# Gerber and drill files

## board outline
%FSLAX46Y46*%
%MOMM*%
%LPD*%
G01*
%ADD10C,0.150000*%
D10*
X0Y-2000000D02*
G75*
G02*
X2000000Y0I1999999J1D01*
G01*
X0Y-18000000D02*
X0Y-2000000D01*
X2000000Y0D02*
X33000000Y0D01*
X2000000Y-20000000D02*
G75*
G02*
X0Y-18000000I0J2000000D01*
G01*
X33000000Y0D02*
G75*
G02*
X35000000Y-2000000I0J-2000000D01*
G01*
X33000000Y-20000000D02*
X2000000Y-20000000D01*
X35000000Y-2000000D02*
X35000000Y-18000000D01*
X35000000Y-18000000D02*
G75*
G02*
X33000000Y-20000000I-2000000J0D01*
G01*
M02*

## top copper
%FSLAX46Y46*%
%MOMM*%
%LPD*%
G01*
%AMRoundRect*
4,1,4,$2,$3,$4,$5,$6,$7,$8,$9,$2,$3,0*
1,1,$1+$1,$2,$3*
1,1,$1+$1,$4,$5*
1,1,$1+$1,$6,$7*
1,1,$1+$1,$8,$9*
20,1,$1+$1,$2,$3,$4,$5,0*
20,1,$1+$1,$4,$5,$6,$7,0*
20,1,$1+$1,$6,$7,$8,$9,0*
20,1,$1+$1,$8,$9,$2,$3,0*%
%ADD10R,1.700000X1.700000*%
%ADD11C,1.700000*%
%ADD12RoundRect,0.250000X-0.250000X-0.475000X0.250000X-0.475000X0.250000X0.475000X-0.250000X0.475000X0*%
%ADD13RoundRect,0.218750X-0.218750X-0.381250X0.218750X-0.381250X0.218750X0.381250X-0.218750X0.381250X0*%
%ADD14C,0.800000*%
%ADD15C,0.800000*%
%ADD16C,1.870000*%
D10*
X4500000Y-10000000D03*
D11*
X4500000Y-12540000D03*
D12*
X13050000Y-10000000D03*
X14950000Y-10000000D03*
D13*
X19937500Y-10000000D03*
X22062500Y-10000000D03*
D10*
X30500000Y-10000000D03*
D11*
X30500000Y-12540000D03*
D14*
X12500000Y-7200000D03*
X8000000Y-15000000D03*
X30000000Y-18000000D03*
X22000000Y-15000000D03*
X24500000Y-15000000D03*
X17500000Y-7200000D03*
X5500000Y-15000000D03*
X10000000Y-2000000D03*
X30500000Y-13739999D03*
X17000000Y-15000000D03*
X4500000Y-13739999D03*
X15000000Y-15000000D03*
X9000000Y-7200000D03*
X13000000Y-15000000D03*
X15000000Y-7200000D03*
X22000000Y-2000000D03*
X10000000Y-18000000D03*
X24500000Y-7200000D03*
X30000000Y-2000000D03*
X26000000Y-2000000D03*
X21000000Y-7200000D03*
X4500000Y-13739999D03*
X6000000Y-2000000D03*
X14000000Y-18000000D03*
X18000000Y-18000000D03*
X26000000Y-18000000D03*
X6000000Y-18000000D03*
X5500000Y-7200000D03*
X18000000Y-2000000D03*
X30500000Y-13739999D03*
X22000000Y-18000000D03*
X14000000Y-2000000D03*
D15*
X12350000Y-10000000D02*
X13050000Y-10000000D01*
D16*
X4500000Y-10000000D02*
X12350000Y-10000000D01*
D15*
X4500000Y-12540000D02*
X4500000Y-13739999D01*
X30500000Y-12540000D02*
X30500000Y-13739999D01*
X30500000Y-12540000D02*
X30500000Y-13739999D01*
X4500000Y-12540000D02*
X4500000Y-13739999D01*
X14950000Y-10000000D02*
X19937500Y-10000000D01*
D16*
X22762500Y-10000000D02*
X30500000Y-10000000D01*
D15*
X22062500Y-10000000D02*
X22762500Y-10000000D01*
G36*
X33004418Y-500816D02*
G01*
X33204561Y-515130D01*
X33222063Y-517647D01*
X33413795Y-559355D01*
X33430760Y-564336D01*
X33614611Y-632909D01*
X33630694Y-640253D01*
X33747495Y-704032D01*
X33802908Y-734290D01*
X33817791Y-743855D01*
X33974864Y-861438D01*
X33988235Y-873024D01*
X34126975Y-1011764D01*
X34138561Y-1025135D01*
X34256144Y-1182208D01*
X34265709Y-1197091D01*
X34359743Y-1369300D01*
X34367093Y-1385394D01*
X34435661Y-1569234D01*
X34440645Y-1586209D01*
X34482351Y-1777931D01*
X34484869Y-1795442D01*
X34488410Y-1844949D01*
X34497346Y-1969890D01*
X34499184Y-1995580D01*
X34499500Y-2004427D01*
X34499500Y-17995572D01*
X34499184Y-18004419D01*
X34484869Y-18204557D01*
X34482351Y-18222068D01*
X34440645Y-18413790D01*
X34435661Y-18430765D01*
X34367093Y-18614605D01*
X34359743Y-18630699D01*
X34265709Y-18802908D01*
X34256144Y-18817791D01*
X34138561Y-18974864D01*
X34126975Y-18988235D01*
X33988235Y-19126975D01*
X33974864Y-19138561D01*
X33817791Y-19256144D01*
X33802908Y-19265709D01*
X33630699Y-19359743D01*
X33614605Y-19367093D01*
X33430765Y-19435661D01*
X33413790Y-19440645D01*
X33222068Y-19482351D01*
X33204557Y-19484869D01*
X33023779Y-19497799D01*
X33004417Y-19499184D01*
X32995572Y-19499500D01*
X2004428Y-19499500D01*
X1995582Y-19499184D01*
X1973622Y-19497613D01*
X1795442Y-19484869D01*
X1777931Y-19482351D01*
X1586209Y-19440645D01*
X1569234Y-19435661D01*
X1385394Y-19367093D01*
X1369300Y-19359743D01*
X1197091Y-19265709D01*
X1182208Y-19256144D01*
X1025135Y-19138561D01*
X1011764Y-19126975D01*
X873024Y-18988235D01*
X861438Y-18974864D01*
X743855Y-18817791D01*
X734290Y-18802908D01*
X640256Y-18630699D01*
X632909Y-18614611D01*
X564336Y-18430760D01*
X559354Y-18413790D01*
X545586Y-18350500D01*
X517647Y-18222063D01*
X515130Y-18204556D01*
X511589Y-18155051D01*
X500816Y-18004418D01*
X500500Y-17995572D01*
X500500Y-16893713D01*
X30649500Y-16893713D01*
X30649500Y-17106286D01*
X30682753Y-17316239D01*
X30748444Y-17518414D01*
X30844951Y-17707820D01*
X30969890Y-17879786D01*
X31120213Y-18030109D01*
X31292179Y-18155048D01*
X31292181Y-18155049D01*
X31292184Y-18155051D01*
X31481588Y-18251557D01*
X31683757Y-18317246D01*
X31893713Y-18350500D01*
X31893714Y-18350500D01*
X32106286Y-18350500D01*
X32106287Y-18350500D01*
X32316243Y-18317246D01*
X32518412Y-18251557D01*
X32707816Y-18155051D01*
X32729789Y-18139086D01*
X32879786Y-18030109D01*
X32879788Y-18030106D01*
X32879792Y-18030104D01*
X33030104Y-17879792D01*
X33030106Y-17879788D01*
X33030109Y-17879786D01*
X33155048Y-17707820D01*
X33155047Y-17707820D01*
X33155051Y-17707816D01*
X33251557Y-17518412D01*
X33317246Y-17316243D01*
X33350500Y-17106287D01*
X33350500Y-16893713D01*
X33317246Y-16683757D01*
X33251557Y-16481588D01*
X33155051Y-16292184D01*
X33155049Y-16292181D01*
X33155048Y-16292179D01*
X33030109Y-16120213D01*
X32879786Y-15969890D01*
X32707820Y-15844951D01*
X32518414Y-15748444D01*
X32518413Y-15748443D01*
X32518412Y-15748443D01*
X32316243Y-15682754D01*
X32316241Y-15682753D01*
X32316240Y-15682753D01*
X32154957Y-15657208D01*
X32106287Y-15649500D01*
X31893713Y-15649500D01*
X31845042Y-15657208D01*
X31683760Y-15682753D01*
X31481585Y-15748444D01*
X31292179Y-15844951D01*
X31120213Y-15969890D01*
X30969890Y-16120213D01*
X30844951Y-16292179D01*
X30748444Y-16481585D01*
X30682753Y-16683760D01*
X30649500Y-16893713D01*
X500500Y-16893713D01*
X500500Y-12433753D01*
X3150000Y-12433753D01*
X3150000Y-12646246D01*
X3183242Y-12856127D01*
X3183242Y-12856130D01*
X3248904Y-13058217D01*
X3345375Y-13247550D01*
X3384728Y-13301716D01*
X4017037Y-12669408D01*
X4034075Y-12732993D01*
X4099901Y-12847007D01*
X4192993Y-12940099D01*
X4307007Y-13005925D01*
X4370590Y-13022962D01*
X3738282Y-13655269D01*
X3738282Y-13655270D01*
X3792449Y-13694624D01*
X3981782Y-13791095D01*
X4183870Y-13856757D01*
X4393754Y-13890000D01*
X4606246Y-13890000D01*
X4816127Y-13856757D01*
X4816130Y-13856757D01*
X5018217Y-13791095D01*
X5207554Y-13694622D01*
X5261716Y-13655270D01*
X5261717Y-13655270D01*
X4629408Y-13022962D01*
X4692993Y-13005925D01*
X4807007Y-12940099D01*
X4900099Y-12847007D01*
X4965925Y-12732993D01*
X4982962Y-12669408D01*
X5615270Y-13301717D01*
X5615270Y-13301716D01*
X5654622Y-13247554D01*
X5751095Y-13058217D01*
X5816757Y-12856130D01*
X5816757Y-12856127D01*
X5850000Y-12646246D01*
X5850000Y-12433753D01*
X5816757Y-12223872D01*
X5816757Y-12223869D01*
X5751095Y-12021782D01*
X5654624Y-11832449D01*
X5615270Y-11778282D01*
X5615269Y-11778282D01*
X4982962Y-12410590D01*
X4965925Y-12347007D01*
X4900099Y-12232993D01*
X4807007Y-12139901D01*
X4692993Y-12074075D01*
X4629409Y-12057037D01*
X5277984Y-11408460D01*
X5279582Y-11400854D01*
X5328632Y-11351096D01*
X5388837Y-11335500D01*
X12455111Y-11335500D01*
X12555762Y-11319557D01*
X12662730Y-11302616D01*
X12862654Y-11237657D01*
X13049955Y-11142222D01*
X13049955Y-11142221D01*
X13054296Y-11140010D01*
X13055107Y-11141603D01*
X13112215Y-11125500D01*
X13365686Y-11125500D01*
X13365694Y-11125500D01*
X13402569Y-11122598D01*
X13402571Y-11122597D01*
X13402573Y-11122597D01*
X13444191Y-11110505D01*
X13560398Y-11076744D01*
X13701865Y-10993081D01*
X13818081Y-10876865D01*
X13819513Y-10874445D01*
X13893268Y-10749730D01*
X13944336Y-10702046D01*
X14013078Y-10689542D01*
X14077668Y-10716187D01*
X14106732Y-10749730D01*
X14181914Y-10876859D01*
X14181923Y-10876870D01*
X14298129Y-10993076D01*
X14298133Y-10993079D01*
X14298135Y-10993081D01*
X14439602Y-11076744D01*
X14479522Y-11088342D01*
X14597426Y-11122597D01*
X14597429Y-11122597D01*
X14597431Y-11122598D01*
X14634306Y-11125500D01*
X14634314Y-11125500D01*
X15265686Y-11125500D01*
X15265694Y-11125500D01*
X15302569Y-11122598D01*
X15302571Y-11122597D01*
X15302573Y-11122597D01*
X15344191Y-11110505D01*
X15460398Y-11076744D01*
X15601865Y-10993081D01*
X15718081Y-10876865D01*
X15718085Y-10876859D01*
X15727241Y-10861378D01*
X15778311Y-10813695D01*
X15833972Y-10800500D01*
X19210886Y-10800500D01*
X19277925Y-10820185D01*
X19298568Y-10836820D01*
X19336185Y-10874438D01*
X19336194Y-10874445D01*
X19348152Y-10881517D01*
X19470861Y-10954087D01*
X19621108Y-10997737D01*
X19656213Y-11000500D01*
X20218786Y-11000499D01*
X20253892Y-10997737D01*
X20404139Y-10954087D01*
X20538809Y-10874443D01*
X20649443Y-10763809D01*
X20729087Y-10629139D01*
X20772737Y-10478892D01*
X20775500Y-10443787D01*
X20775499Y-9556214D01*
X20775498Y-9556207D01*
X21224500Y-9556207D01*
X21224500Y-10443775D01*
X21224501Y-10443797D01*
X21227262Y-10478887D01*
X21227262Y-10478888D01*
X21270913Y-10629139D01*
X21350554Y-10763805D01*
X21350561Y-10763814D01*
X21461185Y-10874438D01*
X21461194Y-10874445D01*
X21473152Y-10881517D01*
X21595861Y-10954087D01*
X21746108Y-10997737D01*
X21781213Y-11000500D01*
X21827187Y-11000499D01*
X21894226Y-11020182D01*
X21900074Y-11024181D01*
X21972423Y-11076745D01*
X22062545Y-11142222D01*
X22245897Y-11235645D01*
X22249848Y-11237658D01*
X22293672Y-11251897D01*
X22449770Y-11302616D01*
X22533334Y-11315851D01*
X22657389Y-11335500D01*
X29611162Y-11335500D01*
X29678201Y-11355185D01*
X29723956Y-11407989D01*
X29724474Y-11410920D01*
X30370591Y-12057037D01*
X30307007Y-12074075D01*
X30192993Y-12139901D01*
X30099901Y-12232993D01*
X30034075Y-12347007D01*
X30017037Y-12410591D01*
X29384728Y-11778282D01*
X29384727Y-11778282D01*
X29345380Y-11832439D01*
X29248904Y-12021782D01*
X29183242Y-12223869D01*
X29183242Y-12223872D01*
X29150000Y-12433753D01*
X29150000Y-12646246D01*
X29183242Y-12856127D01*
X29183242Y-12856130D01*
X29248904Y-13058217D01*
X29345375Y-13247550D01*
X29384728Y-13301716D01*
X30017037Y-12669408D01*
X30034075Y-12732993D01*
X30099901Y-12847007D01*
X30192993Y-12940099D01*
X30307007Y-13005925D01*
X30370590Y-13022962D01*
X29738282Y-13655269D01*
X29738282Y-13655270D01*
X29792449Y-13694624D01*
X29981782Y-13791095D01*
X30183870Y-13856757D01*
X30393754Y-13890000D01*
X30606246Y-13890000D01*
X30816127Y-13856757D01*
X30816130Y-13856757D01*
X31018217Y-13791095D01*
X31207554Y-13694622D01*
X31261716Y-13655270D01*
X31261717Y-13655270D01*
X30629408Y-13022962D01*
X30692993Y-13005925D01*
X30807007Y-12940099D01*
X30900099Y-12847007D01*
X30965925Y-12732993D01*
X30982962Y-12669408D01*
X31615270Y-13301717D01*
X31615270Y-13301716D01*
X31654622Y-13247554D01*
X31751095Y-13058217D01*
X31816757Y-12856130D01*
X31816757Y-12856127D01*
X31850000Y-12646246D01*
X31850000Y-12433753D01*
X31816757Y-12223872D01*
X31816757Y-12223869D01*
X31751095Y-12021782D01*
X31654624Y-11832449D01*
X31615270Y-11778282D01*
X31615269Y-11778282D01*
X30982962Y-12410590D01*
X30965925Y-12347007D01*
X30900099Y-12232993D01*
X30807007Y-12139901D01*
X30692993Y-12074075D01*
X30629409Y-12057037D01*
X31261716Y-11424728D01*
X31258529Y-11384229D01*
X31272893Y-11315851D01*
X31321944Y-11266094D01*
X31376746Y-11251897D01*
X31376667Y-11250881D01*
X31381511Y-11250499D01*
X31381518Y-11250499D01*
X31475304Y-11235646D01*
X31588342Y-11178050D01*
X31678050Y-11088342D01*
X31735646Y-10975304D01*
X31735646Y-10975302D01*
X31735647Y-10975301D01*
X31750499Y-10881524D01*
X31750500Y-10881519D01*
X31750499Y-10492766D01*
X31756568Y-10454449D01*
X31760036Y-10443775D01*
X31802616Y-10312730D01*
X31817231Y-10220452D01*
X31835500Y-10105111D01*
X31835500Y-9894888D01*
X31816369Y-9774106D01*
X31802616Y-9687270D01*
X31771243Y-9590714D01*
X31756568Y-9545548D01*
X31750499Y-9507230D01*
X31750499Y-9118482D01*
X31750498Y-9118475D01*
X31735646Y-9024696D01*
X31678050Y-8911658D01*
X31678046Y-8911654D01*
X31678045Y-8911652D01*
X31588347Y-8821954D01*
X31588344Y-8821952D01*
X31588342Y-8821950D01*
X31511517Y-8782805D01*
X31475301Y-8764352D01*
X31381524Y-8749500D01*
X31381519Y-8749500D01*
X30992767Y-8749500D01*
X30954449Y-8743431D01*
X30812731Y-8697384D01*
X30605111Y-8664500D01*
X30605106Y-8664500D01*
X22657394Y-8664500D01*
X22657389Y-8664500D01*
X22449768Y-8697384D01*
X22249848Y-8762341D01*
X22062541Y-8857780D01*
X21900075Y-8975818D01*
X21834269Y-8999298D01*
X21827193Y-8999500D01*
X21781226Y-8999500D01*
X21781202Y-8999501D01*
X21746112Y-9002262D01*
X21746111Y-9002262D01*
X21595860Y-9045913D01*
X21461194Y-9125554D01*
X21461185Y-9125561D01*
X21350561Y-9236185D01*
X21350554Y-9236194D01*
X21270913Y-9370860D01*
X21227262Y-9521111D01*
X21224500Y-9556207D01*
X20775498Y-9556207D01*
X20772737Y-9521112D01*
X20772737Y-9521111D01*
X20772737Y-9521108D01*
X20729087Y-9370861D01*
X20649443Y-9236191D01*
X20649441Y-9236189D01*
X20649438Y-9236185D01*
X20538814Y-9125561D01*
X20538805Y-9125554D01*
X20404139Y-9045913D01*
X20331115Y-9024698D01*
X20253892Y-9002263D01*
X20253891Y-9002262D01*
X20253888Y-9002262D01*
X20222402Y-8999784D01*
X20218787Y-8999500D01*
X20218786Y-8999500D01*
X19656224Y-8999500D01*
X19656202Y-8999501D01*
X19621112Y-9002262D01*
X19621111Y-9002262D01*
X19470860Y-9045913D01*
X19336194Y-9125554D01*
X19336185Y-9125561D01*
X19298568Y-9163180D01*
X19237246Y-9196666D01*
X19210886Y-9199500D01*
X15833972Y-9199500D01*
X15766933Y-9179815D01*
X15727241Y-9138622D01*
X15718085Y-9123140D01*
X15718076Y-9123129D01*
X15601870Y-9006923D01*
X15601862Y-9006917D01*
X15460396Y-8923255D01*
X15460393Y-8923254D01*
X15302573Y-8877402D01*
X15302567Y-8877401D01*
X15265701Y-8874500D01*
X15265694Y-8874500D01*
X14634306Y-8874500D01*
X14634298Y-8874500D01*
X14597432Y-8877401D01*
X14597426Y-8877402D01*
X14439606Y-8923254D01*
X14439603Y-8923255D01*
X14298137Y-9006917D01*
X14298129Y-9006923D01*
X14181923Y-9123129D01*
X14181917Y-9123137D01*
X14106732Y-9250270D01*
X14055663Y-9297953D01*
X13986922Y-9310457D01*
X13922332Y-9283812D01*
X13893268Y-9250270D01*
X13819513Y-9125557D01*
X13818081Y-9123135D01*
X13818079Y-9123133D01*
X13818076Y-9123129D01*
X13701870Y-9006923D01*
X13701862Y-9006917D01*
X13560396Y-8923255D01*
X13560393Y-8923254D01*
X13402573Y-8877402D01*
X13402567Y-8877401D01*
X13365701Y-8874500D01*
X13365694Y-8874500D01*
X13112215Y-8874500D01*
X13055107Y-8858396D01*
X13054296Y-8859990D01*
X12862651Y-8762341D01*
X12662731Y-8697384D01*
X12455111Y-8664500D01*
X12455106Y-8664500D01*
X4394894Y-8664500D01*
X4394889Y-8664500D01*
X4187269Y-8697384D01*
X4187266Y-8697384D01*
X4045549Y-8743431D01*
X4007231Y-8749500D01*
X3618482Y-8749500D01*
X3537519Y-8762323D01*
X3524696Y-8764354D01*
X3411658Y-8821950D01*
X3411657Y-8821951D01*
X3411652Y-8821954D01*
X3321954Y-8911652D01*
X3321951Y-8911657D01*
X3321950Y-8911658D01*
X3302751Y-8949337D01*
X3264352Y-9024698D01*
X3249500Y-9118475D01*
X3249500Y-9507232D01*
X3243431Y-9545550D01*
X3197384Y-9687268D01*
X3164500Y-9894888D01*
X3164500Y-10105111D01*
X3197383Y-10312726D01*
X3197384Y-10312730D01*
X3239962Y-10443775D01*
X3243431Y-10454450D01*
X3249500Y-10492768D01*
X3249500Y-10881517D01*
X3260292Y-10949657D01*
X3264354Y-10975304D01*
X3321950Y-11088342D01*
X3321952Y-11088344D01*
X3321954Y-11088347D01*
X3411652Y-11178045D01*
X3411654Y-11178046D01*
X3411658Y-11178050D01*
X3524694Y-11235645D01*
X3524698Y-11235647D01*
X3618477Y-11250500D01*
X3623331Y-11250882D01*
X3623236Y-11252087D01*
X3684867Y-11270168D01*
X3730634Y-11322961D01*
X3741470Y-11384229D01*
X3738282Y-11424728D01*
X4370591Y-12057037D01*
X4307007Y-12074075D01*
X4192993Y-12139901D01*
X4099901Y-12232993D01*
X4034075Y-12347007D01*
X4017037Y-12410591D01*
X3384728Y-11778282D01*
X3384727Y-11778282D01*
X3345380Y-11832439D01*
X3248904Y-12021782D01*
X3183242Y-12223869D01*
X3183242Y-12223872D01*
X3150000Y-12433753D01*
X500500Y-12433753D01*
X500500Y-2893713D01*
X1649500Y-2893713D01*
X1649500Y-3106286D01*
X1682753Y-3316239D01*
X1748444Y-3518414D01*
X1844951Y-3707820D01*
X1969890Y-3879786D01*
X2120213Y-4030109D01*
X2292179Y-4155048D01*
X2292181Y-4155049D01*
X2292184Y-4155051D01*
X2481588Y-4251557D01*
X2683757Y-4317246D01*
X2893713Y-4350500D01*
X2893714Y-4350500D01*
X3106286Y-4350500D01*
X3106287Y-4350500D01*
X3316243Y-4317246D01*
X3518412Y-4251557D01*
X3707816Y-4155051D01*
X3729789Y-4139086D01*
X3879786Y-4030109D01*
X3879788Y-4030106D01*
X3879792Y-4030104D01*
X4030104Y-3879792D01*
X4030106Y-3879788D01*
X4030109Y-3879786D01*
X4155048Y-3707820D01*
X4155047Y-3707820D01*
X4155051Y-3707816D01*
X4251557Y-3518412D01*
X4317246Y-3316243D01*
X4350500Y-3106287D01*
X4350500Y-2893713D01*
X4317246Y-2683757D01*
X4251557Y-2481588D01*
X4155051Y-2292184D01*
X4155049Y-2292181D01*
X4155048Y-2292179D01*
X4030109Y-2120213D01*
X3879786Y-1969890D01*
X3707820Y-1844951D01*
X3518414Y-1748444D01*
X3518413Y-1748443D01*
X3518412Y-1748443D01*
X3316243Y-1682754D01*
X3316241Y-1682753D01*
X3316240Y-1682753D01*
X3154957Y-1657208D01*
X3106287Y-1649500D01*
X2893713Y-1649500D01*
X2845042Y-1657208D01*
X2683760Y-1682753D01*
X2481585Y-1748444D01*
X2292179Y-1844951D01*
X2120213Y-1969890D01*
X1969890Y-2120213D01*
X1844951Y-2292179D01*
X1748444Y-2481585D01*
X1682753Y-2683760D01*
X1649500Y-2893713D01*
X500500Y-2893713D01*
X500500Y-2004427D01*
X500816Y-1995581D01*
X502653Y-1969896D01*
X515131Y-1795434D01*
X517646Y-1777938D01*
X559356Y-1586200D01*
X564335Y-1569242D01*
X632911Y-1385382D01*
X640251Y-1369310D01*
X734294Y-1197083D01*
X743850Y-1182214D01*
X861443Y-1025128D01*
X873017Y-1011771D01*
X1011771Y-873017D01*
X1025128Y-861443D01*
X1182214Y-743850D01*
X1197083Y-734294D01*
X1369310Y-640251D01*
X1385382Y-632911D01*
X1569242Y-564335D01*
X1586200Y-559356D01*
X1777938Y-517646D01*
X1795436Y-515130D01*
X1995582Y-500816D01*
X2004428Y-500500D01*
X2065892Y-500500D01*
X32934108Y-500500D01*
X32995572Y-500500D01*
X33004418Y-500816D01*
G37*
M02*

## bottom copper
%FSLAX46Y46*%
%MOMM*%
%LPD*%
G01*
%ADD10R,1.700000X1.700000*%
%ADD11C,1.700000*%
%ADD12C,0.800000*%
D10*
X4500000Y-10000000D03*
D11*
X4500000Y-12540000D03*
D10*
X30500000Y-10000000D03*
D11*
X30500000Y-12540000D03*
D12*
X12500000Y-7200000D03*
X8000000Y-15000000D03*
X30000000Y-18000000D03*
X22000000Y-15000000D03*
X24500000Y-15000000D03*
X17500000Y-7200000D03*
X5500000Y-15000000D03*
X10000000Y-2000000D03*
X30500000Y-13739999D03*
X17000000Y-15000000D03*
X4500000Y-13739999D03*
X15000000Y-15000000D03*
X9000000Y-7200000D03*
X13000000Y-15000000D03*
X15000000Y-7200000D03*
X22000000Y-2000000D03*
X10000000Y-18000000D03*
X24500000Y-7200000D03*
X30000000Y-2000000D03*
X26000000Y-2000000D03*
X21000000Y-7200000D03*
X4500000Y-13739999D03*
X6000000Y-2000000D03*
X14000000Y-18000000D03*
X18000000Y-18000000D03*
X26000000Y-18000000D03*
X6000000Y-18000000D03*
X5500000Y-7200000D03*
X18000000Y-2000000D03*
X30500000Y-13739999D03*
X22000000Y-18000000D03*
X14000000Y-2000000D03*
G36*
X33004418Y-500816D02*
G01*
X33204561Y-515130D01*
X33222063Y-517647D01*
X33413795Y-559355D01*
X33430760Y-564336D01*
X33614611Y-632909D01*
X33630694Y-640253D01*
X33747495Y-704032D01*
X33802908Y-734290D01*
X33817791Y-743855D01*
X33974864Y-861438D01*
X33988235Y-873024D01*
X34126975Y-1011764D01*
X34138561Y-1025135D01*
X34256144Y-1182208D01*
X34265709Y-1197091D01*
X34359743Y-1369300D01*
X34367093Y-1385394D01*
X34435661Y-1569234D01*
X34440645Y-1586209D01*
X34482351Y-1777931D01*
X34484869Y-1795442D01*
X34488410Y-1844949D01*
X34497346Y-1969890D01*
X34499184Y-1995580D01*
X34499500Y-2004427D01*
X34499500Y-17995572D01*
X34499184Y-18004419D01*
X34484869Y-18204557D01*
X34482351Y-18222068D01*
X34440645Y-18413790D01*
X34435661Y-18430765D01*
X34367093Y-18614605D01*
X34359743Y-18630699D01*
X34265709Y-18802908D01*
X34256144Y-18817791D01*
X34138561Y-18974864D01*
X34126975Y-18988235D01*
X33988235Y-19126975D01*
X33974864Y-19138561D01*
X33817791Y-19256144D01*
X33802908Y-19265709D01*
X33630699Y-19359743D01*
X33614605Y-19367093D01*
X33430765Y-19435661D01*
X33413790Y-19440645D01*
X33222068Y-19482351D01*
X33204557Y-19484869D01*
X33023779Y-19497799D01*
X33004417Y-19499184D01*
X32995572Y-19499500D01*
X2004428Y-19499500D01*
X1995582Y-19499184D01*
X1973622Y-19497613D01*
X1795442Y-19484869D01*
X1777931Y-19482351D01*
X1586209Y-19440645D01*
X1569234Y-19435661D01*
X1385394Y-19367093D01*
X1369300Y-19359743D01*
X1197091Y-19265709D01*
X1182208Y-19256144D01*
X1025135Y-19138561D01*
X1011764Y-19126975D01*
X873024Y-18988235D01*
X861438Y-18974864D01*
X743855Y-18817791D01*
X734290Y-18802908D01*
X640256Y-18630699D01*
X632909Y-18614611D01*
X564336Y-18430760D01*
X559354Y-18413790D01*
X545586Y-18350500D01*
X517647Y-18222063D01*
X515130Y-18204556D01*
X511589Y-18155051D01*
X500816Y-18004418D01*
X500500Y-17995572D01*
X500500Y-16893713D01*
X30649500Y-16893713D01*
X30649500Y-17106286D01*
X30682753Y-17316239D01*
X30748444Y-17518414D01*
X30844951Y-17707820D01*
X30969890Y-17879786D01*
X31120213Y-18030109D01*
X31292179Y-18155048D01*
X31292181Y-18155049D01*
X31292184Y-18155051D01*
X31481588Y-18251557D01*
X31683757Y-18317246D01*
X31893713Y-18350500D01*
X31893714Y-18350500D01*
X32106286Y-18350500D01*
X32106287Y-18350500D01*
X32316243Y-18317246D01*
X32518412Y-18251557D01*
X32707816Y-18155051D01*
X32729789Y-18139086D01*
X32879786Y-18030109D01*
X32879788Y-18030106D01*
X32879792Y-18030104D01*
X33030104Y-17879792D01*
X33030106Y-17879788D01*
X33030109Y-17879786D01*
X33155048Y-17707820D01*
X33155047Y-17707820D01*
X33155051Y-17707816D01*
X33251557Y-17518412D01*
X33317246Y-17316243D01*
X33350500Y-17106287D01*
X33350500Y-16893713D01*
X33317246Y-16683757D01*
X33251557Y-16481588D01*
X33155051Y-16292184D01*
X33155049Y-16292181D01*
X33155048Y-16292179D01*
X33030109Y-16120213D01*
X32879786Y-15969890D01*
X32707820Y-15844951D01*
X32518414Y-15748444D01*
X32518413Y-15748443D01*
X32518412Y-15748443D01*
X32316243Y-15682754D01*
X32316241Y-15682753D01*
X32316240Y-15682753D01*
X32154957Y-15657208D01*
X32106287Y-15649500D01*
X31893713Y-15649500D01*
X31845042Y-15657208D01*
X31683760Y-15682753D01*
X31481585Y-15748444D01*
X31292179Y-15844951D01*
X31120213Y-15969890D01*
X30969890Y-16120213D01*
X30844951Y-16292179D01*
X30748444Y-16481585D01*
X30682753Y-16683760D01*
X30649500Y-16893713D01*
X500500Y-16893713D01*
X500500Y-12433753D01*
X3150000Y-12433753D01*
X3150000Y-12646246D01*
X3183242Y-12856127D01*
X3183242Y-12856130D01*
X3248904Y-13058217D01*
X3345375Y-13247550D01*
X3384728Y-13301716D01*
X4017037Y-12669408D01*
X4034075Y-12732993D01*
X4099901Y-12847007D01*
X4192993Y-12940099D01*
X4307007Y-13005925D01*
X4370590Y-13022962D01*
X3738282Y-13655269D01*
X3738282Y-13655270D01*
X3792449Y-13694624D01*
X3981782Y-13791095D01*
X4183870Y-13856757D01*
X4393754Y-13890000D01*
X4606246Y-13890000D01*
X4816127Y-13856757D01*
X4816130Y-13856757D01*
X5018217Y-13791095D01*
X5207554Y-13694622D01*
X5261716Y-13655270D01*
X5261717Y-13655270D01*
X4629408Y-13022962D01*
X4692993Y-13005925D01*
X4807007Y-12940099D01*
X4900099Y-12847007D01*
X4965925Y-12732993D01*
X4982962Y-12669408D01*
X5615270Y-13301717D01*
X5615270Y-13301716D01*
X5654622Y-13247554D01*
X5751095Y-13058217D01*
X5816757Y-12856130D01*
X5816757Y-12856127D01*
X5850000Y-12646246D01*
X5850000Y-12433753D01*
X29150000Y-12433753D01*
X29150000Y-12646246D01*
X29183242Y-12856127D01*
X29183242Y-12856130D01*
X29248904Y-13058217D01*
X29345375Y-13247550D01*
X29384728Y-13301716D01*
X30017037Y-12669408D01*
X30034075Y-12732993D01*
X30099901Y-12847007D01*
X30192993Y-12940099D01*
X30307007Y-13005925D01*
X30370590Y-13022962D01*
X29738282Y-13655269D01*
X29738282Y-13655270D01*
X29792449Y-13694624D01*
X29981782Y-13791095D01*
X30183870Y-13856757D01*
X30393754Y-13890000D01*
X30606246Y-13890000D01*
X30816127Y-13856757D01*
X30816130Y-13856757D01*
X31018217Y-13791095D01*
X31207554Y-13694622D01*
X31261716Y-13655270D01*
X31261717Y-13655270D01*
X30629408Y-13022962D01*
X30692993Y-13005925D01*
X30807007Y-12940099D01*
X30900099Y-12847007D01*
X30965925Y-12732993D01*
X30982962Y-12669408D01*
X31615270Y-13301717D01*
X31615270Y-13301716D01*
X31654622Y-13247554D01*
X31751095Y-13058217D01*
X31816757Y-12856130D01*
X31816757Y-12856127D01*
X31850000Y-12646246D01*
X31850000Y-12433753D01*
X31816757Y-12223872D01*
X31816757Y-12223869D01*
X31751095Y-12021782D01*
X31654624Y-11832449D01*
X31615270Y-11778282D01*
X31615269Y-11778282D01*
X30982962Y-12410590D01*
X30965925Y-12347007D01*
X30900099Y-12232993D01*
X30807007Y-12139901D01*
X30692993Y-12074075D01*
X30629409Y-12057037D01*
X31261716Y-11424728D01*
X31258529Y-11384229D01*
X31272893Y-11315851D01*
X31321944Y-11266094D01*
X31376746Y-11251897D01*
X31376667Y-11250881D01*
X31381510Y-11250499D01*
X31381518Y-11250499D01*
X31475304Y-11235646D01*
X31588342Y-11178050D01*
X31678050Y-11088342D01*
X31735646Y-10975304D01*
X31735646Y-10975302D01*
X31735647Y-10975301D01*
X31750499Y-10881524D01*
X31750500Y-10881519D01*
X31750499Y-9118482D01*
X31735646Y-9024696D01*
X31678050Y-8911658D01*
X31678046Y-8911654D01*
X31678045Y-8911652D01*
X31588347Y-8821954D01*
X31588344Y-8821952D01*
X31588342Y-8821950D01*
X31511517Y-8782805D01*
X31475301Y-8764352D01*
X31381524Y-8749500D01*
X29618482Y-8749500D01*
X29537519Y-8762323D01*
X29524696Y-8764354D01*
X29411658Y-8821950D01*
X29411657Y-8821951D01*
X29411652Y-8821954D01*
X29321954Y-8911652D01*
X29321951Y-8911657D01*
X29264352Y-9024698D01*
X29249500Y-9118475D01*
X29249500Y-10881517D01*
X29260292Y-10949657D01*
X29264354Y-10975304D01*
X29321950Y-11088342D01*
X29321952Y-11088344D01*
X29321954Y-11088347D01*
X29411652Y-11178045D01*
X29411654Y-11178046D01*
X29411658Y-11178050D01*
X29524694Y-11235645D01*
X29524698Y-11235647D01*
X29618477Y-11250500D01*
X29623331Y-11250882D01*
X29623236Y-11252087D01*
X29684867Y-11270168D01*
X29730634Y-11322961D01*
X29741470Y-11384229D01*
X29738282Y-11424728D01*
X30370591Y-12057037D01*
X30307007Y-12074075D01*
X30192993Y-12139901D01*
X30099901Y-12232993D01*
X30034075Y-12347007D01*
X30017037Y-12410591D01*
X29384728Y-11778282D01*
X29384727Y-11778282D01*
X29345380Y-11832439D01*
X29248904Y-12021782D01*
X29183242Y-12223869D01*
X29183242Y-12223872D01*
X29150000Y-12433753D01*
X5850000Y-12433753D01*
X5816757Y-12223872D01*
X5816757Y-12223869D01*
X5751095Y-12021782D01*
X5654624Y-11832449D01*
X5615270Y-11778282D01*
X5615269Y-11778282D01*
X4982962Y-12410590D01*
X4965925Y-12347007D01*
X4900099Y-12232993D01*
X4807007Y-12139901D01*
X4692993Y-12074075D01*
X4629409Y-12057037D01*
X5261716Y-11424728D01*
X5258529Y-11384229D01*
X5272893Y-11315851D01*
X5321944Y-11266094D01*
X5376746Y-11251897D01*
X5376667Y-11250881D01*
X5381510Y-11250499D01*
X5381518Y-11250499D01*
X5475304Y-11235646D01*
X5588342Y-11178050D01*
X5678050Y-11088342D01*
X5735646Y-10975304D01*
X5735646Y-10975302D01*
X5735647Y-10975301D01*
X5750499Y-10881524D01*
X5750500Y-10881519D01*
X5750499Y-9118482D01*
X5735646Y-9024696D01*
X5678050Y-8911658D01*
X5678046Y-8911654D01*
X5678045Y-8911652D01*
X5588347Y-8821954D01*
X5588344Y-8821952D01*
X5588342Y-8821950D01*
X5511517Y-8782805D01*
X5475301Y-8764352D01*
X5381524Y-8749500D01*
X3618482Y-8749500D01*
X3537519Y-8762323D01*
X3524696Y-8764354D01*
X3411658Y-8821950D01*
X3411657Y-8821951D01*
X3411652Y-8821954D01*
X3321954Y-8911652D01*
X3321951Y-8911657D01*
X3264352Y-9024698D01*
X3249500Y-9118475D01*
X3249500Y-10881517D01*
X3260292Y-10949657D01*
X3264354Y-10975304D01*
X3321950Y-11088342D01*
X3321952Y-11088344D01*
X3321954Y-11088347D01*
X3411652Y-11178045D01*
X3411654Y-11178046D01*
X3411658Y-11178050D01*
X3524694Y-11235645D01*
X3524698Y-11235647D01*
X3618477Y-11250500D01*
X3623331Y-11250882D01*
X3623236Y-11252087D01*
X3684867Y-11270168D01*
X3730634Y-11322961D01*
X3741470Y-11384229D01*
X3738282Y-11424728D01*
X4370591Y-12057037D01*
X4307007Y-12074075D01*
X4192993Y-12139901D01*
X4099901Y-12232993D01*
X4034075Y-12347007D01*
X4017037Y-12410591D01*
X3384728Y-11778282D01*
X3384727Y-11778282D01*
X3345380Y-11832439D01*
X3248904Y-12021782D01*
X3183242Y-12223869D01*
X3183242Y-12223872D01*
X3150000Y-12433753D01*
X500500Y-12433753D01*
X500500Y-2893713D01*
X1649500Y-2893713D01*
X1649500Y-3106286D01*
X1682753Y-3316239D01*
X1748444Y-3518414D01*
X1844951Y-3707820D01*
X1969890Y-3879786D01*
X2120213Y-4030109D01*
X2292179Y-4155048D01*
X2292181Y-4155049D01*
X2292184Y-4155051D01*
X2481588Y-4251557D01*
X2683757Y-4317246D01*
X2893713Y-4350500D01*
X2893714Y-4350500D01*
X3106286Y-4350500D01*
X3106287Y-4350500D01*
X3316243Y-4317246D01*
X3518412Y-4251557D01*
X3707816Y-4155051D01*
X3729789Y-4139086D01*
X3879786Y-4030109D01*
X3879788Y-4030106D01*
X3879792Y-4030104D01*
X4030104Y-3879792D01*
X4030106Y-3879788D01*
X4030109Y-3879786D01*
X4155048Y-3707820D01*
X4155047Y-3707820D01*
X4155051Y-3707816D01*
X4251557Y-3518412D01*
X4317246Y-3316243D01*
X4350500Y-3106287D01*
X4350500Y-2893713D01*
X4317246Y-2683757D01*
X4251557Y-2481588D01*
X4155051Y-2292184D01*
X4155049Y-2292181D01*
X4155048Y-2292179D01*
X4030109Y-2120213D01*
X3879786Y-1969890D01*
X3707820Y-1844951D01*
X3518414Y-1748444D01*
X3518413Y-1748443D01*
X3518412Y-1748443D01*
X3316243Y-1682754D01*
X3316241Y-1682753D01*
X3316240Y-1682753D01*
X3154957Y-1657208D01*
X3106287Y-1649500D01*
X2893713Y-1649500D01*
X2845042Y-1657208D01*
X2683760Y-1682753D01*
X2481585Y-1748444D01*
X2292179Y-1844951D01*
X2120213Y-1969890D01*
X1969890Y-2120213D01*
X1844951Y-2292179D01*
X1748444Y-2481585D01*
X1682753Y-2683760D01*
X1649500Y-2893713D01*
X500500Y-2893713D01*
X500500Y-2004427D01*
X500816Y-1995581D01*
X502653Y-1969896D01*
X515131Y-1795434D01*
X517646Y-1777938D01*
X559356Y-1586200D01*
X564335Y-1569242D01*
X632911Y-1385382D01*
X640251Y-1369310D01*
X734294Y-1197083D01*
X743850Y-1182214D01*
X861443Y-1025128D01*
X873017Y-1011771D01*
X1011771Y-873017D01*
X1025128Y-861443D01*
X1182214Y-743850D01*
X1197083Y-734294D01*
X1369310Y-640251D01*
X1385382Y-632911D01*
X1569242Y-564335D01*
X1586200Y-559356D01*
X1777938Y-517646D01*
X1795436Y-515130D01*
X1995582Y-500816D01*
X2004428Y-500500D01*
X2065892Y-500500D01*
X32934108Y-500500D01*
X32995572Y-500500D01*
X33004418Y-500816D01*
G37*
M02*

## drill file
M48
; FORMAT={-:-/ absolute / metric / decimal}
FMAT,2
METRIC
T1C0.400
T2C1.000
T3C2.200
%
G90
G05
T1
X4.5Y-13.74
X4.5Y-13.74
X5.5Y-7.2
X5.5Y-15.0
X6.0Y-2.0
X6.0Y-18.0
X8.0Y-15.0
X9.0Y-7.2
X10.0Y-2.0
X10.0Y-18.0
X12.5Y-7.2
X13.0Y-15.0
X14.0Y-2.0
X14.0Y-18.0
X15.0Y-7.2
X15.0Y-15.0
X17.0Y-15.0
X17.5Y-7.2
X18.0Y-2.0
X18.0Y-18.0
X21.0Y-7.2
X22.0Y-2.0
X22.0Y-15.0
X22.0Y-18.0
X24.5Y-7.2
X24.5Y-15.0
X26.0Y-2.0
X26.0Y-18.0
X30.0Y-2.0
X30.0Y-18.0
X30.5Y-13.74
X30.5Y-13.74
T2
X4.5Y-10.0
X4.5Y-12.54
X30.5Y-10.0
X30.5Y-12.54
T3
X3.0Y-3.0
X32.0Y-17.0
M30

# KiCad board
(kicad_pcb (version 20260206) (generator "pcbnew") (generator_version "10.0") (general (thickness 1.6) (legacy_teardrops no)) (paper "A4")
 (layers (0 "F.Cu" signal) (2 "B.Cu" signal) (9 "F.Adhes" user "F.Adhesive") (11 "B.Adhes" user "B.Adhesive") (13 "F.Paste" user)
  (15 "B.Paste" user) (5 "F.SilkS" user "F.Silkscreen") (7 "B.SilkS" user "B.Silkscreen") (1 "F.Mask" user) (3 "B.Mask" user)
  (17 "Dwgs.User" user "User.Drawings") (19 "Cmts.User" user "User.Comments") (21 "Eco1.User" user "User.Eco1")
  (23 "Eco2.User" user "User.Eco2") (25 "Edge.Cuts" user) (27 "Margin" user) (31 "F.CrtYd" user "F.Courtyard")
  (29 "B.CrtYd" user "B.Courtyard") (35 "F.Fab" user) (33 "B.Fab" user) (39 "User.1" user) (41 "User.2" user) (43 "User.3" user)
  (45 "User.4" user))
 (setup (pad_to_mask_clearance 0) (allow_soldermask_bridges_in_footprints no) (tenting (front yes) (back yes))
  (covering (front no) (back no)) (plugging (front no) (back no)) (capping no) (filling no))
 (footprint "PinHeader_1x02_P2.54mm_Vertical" (layer "F.Cu") (at 4.5 10)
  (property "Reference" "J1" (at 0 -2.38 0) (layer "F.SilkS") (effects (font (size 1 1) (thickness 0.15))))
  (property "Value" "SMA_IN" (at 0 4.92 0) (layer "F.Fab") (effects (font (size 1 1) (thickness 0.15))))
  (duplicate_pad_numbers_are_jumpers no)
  (pad "1" thru_hole rect (at 0 0) (size 1.7 1.7) (drill 1) (layers "*.Cu" "*.Mask") (remove_unused_layers no) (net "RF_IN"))
  (pad "2" thru_hole circle (at 0 2.54) (size 1.7 1.7) (drill 1) (layers "*.Cu" "*.Mask") (remove_unused_layers no) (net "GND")))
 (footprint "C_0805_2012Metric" (layer "F.Cu") (at 14 10)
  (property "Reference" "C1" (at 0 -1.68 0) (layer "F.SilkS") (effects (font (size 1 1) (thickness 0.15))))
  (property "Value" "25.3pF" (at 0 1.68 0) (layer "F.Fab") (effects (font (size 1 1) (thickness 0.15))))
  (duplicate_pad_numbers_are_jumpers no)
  (pad "1" smd roundrect (at -0.95 0) (size 1 1.45) (layers "F.Cu" "F.Mask" "F.Paste") (roundrect_rratio 0.25) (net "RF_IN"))
  (pad "2" smd roundrect (at 0.95 0) (size 1 1.45) (layers "F.Cu" "F.Mask" "F.Paste") (roundrect_rratio 0.25) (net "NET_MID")))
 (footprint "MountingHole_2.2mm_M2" (layer "F.Cu") (at 32 17)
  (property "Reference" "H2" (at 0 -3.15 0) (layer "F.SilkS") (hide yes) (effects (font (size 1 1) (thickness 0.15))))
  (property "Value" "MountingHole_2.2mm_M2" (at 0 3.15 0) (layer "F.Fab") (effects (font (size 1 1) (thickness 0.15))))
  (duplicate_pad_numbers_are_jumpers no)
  (pad "" np_thru_hole circle (at 0 0) (size 2.2 2.2) (drill 2.2) (layers "*.Cu" "*.Mask")))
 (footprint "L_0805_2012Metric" (layer "F.Cu") (at 21 10)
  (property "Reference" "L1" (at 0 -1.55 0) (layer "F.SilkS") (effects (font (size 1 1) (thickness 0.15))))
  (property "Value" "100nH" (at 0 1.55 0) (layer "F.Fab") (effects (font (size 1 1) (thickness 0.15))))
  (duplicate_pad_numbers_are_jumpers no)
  (pad "1" smd roundrect (at -1.0625 0) (size 0.875 1.2) (layers "F.Cu" "F.Mask" "F.Paste") (roundrect_rratio 0.25) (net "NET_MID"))
  (pad "2" smd roundrect (at 1.0625 0) (size 0.875 1.2) (layers "F.Cu" "F.Mask" "F.Paste") (roundrect_rratio 0.25) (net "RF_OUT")))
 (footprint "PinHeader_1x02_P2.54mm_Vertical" (layer "F.Cu") (at 30.5 10)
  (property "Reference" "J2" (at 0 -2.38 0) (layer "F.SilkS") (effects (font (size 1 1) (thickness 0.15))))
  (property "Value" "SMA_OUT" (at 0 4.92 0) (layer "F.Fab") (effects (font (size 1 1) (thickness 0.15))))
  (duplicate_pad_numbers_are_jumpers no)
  (pad "1" thru_hole rect (at 0 0) (size 1.7 1.7) (drill 1) (layers "*.Cu" "*.Mask") (remove_unused_layers no) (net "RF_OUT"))
  (pad "2" thru_hole circle (at 0 2.54) (size 1.7 1.7) (drill 1) (layers "*.Cu" "*.Mask") (remove_unused_layers no) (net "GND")))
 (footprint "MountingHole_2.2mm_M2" (layer "F.Cu") (at 3 3)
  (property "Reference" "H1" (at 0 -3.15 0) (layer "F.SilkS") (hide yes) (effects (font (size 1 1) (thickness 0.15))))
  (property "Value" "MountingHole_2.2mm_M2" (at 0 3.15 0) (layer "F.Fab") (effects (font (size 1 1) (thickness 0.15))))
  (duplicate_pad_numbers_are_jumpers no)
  (pad "" np_thru_hole circle (at 0 0) (size 2.2 2.2) (drill 2.2) (layers "*.Cu" "*.Mask")))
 (gr_arc (start 0 2) (mid 0.585786 0.585786) (end 2 0) (stroke (width 0.15) (type default)) (layer "Edge.Cuts"))
 (gr_line (start 0 18) (end 0 2) (stroke (width 0.15) (type default)) (layer "Edge.Cuts"))
 (gr_line (start 2 0) (end 33 0) (stroke (width 0.15) (type default)) (layer "Edge.Cuts"))
 (gr_arc (start 2 20) (mid 0.585786 19.414214) (end 0 18) (stroke (width 0.15) (type default)) (layer "Edge.Cuts"))
 (gr_arc (start 33 0) (mid 34.414214 0.585786) (end 35 2) (stroke (width 0.15) (type default)) (layer "Edge.Cuts"))
 (gr_line (start 33 20) (end 2 20) (stroke (width 0.15) (type default)) (layer "Edge.Cuts"))
 (gr_line (start 35 2) (end 35 18) (stroke (width 0.15) (type default)) (layer "Edge.Cuts"))
 (gr_arc (start 35 18) (mid 34.414214 19.414214) (end 33 20) (stroke (width 0.15) (type default)) (layer "Edge.Cuts"))
 (segment (start 12.35 10) (end 13.05 10) (width 0.8) (layer "F.Cu") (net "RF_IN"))
 (segment (start 4.5 10) (end 12.35 10) (width 1.87) (layer "F.Cu") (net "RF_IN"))
 (segment (start 4.5 12.54) (end 4.5 13.739999) (width 0.8) (layer "F.Cu") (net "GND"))
 (segment (start 30.5 12.54) (end 30.5 13.739999) (width 0.8) (layer "F.Cu") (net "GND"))
 (segment (start 30.5 12.54) (end 30.5 13.739999) (width 0.8) (layer "F.Cu") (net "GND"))
 (segment (start 4.5 12.54) (end 4.5 13.739999) (width 0.8) (layer "F.Cu") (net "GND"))
 (via (at 12.5 7.2) (size 0.8) (drill 0.4) (layers "F.Cu" "B.Cu") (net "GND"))
 (via (at 8 15) (size 0.8) (drill 0.4) (layers "F.Cu" "B.Cu") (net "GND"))
 (via (at 30 18) (size 0.8) (drill 0.4) (layers "F.Cu" "B.Cu") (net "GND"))
 (via (at 22 15) (size 0.8) (drill 0.4) (layers "F.Cu" "B.Cu") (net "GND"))
 (via (at 24.5 15) (size 0.8) (drill 0.4) (layers "F.Cu" "B.Cu") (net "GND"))
 (via (at 17.5 7.2) (size 0.8) (drill 0.4) (layers "F.Cu" "B.Cu") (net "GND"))
 (via (at 5.5 15) (size 0.8) (drill 0.4) (layers "F.Cu" "B.Cu") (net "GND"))
 (via (at 10 2) (size 0.8) (drill 0.4) (layers "F.Cu" "B.Cu") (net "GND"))
 (via (at 30.5 13.739999) (size 0.8) (drill 0.4) (layers "F.Cu" "B.Cu") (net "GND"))
 (via (at 17 15) (size 0.8) (drill 0.4) (layers "F.Cu" "B.Cu") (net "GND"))
 (via (at 4.5 13.739999) (size 0.8) (drill 0.4) (layers "F.Cu" "B.Cu") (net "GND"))
 (via (at 15 15) (size 0.8) (drill 0.4) (layers "F.Cu" "B.Cu") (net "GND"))
 (via (at 9 7.2) (size 0.8) (drill 0.4) (layers "F.Cu" "B.Cu") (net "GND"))
 (via (at 13 15) (size 0.8) (drill 0.4) (layers "F.Cu" "B.Cu") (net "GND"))
 (via (at 15 7.2) (size 0.8) (drill 0.4) (layers "F.Cu" "B.Cu") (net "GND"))
 (via (at 22 2) (size 0.8) (drill 0.4) (layers "F.Cu" "B.Cu") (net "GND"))
 (via (at 10 18) (size 0.8) (drill 0.4) (layers "F.Cu" "B.Cu") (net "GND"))
 (via (at 24.5 7.2) (size 0.8) (drill 0.4) (layers "F.Cu" "B.Cu") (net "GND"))
 (via (at 30 2) (size 0.8) (drill 0.4) (layers "F.Cu" "B.Cu") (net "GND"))
 (via (at 26 2) (size 0.8) (drill 0.4) (layers "F.Cu" "B.Cu") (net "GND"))
 (via (at 21 7.2) (size 0.8) (drill 0.4) (layers "F.Cu" "B.Cu") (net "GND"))
 (via (at 4.5 13.739999) (size 0.8) (drill 0.4) (layers "F.Cu" "B.Cu") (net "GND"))
 (via (at 6 2) (size 0.8) (drill 0.4) (layers "F.Cu" "B.Cu") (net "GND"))
 (via (at 14 18) (size 0.8) (drill 0.4) (layers "F.Cu" "B.Cu") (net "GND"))
 (via (at 18 18) (size 0.8) (drill 0.4) (layers "F.Cu" "B.Cu") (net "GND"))
 (via (at 26 18) (size 0.8) (drill 0.4) (layers "F.Cu" "B.Cu") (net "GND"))
 (via (at 6 18) (size 0.8) (drill 0.4) (layers "F.Cu" "B.Cu") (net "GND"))
 (via (at 5.5 7.2) (size 0.8) (drill 0.4) (layers "F.Cu" "B.Cu") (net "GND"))
 (via (at 18 2) (size 0.8) (drill 0.4) (layers "F.Cu" "B.Cu") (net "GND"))
 (via (at 30.5 13.739999) (size 0.8) (drill 0.4) (layers "F.Cu" "B.Cu") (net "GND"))
 (via (at 22 18) (size 0.8) (drill 0.4) (layers "F.Cu" "B.Cu") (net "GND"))
 (via (at 14 2) (size 0.8) (drill 0.4) (layers "F.Cu" "B.Cu") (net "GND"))
 (segment (start 14.95 10) (end 19.9375 10) (width 0.8) (layer "F.Cu") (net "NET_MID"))
 (segment (start 22.7625 10) (end 30.5 10) (width 1.87) (layer "F.Cu") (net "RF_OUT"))
 (segment (start 22.0625 10) (end 22.7625 10) (width 0.8) (layer "F.Cu") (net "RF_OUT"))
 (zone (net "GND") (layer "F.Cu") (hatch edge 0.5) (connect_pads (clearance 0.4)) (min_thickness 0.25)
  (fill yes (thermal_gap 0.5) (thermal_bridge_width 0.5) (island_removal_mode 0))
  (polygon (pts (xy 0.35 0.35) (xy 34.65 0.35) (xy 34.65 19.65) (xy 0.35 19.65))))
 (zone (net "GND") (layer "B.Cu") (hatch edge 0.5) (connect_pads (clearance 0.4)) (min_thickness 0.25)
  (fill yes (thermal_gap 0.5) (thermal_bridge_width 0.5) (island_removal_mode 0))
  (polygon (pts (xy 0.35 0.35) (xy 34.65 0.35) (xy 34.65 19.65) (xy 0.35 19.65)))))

